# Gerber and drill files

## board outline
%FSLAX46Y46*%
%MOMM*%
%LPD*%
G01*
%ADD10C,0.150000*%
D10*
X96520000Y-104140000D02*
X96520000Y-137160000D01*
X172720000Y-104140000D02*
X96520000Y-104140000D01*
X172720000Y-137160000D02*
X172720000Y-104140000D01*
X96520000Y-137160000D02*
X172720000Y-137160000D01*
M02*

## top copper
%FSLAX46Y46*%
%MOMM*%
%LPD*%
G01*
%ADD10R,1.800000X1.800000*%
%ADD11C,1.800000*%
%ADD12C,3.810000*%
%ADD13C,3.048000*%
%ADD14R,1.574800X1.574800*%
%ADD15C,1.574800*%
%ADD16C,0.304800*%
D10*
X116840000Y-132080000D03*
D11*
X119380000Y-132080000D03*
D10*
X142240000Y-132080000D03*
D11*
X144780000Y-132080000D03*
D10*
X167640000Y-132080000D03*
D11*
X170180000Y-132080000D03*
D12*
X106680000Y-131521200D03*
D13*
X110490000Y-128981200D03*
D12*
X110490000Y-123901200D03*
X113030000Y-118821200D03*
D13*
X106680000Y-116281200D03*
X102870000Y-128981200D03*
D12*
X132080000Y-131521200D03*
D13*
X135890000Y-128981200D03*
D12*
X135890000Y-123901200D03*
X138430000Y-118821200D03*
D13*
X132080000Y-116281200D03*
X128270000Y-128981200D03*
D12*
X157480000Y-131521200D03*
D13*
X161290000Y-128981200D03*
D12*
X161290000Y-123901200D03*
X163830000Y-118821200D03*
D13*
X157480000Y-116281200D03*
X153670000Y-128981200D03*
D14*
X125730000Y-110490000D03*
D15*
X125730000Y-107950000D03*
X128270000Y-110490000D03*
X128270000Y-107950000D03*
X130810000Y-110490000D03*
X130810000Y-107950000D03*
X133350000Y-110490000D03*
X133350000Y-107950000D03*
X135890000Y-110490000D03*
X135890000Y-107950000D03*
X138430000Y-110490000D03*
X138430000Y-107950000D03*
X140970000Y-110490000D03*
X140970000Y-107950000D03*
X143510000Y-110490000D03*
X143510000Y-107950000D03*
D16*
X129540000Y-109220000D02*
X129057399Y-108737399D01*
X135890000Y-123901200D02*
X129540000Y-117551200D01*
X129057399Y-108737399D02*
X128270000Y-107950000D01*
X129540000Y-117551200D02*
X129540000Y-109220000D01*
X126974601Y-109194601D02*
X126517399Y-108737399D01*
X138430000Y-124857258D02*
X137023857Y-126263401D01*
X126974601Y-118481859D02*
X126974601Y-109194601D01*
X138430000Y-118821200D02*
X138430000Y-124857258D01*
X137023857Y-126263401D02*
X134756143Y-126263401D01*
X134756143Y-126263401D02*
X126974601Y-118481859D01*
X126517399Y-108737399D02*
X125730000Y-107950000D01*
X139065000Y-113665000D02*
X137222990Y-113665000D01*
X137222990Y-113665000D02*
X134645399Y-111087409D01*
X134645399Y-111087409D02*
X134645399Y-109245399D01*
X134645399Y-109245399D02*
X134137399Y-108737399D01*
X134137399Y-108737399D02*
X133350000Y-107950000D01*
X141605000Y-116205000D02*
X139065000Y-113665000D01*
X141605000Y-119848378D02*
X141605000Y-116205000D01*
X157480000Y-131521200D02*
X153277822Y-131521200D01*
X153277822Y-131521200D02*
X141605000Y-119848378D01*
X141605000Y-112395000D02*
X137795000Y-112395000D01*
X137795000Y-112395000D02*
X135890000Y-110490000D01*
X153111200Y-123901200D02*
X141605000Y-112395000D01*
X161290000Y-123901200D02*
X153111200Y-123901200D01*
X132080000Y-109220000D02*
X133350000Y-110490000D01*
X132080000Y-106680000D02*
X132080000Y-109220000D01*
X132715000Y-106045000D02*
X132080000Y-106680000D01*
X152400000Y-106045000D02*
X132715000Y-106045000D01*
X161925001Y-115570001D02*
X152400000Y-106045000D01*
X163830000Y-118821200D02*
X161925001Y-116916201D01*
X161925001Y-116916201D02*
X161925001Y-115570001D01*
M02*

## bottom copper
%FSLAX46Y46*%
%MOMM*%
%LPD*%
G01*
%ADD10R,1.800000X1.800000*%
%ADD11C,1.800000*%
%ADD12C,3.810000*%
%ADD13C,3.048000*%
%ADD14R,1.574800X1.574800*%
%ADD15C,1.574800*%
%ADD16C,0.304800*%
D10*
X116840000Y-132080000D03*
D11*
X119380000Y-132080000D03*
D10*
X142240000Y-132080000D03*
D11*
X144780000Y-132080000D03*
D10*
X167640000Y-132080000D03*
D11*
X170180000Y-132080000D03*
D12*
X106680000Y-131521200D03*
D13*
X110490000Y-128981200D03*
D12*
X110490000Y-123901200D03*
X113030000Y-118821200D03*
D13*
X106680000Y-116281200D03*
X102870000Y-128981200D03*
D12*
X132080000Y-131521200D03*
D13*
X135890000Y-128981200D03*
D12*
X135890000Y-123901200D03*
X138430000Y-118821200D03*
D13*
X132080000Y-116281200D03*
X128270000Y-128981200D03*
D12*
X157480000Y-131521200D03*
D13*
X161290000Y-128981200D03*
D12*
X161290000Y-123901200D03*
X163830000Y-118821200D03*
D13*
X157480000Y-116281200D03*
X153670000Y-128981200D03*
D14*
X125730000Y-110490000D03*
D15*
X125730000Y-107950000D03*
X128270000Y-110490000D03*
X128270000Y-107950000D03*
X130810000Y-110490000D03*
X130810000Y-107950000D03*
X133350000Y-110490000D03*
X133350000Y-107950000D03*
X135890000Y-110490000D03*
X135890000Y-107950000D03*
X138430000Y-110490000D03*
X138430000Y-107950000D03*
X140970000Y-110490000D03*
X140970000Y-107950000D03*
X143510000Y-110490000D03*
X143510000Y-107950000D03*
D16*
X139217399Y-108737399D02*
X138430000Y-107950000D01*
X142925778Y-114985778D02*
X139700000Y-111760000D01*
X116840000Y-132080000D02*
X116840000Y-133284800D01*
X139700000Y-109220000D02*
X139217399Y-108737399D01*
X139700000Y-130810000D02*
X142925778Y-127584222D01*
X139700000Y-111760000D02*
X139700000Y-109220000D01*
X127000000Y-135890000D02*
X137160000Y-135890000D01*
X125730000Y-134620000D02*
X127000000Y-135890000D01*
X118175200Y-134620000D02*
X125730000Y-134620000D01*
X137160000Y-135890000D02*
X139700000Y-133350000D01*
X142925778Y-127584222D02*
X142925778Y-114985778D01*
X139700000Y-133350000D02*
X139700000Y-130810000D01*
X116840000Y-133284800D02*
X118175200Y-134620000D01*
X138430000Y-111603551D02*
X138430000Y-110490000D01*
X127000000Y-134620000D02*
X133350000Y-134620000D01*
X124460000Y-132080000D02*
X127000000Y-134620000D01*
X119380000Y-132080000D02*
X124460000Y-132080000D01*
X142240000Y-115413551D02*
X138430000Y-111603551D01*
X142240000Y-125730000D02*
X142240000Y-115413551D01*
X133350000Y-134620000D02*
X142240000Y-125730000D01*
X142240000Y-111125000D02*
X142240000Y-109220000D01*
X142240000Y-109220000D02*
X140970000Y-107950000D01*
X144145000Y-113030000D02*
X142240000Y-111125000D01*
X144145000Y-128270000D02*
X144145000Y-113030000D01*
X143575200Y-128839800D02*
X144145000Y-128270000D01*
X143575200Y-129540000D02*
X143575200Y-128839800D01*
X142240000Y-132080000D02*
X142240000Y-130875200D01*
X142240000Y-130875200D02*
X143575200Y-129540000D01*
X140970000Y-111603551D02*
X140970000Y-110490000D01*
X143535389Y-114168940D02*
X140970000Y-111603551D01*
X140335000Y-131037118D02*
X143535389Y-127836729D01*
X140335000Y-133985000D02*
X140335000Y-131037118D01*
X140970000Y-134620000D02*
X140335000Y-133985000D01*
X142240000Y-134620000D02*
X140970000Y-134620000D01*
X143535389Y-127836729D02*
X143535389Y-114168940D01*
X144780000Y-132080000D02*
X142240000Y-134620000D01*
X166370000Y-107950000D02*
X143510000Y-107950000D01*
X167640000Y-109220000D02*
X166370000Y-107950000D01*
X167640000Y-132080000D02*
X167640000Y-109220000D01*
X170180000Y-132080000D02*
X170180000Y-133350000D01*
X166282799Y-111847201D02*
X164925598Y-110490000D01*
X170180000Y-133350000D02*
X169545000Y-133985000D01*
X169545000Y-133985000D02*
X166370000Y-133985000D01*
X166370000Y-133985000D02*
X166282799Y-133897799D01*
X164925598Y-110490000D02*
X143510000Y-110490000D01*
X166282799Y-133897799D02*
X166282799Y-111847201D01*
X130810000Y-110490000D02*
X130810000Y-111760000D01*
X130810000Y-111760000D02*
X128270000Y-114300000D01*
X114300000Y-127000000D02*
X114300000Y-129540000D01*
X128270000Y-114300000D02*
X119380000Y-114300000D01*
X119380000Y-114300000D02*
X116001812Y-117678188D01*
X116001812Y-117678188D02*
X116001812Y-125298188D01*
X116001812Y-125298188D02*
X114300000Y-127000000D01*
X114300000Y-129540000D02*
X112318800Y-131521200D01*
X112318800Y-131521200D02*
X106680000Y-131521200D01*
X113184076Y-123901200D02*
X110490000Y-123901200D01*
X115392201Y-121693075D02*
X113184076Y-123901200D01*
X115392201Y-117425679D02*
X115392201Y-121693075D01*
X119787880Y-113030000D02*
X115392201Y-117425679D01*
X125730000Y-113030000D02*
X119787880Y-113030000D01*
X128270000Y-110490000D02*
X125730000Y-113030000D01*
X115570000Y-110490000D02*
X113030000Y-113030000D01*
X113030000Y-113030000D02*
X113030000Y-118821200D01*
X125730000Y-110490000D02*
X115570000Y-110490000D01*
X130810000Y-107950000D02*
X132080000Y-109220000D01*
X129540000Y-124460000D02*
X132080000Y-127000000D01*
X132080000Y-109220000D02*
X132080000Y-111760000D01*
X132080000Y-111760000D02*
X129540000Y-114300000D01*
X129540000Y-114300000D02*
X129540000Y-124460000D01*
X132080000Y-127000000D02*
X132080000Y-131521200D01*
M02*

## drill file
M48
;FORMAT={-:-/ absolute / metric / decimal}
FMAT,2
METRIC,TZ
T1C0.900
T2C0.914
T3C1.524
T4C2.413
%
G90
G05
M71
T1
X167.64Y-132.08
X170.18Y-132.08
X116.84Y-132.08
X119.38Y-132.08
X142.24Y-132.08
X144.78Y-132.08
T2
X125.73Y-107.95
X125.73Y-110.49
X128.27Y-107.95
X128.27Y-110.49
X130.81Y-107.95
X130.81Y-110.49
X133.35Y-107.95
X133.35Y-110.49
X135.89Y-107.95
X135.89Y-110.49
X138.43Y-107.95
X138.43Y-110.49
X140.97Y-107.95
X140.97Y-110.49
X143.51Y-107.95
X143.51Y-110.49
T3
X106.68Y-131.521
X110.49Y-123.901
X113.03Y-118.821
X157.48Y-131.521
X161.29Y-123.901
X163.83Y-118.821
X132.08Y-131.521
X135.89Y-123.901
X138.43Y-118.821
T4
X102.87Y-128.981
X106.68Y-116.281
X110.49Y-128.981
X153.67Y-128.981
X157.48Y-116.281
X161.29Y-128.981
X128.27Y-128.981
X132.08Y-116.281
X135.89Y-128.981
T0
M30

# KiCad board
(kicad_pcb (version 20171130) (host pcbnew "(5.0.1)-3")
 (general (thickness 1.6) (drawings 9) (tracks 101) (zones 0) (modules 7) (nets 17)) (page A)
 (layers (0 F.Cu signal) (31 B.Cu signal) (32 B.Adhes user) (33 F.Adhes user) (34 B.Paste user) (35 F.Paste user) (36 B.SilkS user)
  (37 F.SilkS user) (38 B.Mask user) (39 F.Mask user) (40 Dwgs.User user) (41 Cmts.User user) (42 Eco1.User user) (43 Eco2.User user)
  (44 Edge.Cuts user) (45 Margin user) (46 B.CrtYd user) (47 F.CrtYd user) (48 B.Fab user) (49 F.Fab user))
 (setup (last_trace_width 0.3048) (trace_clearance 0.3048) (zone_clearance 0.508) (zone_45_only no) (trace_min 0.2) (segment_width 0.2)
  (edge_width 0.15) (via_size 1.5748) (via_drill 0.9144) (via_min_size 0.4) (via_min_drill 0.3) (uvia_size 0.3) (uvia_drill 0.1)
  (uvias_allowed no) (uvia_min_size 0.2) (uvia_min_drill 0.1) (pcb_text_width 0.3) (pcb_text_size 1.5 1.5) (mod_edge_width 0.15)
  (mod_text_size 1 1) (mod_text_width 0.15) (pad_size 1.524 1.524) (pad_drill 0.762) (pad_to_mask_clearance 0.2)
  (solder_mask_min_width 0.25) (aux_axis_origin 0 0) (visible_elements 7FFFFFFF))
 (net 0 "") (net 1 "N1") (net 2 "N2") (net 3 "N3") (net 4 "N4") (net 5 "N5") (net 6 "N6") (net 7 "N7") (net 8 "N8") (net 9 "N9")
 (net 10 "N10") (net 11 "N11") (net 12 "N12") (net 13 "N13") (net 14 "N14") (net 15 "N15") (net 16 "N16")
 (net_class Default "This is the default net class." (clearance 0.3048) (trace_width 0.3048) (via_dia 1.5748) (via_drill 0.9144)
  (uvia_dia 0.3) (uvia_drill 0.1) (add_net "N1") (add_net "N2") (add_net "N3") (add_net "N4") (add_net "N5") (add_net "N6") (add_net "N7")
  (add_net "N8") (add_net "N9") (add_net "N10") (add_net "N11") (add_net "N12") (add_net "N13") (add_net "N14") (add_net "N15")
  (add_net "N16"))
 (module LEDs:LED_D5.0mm (layer F.Cu) (at 116.84 132.08)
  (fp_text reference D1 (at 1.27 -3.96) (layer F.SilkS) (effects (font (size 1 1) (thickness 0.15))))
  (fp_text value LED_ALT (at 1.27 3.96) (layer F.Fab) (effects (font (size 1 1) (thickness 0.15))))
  (pad 1 thru_hole rect (at 0 0) (size 1.8 1.8) (drill 0.9) (layers *.Cu *.Mask) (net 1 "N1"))
  (pad 2 thru_hole circle (at 2.54 0) (size 1.8 1.8) (drill 0.9) (layers *.Cu *.Mask) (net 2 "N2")))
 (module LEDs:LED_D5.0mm (layer F.Cu) (at 142.24 132.08)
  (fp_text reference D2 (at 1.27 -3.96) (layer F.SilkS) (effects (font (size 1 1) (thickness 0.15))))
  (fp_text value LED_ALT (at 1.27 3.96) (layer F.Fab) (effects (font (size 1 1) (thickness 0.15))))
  (pad 1 thru_hole rect (at 0 0) (size 1.8 1.8) (drill 0.9) (layers *.Cu *.Mask) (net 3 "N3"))
  (pad 2 thru_hole circle (at 2.54 0) (size 1.8 1.8) (drill 0.9) (layers *.Cu *.Mask) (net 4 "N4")))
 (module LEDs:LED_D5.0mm (layer F.Cu) (at 167.64 132.08)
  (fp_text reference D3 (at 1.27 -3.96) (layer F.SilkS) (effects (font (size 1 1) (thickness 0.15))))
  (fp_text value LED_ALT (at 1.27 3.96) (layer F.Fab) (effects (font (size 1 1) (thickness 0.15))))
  (pad 1 thru_hole rect (at 0 0) (size 1.8 1.8) (drill 0.9) (layers *.Cu *.Mask) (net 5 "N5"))
  (pad 2 thru_hole circle (at 2.54 0) (size 1.8 1.8) (drill 0.9) (layers *.Cu *.Mask) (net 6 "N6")))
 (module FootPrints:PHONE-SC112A (layer F.Cu) (at 106.68 137.16 270)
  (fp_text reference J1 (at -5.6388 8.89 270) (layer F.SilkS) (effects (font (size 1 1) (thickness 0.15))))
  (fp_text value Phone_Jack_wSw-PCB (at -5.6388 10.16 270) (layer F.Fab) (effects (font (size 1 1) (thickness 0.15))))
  (pad 1 thru_hole circle (at -5.6388 0 270) (size 3.81 3.81) (drill 1.524) (layers *.Cu *.Mask F.SilkS) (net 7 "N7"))
  (pad "" thru_hole circle (at -8.1788 -3.81 270) (size 3.048 3.048) (drill 2.413) (layers *.Cu *.Mask F.SilkS))
  (pad 2 thru_hole circle (at -13.2588 -3.81 270) (size 3.81 3.81) (drill 1.524) (layers *.Cu *.Mask F.SilkS) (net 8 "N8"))
  (pad 3 thru_hole circle (at -18.3388 -6.35 270) (size 3.81 3.81) (drill 1.524) (layers *.Cu *.Mask F.SilkS) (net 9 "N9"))
  (pad "" thru_hole circle (at -20.8788 0 270) (size 3.048 3.048) (drill 2.413) (layers *.Cu *.Mask F.SilkS))
  (pad "" thru_hole circle (at -8.1788 3.81 270) (size 3.048 3.048) (drill 2.413) (layers *.Cu *.Mask F.SilkS)))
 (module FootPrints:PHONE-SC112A (layer F.Cu) (at 132.08 137.16 270)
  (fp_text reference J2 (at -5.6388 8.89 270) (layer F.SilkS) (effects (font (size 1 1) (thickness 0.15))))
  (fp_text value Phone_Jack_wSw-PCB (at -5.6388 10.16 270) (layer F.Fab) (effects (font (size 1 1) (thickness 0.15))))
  (pad 1 thru_hole circle (at -5.6388 0 270) (size 3.81 3.81) (drill 1.524) (layers *.Cu *.Mask F.SilkS) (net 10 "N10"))
  (pad "" thru_hole circle (at -8.1788 -3.81 270) (size 3.048 3.048) (drill 2.413) (layers *.Cu *.Mask F.SilkS))
  (pad 2 thru_hole circle (at -13.2588 -3.81 270) (size 3.81 3.81) (drill 1.524) (layers *.Cu *.Mask F.SilkS) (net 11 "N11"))
  (pad 3 thru_hole circle (at -18.3388 -6.35 270) (size 3.81 3.81) (drill 1.524) (layers *.Cu *.Mask F.SilkS) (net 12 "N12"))
  (pad "" thru_hole circle (at -20.8788 0 270) (size 3.048 3.048) (drill 2.413) (layers *.Cu *.Mask F.SilkS))
  (pad "" thru_hole circle (at -8.1788 3.81 270) (size 3.048 3.048) (drill 2.413) (layers *.Cu *.Mask F.SilkS)))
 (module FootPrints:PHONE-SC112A (layer F.Cu) (at 157.48 137.16 270)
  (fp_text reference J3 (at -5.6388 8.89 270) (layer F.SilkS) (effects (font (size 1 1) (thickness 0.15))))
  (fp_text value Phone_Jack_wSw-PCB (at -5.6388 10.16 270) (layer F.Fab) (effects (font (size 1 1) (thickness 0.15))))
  (pad 1 thru_hole circle (at -5.6388 0 270) (size 3.81 3.81) (drill 1.524) (layers *.Cu *.Mask F.SilkS) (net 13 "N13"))
  (pad "" thru_hole circle (at -8.1788 -3.81 270) (size 3.048 3.048) (drill 2.413) (layers *.Cu *.Mask F.SilkS))
  (pad 2 thru_hole circle (at -13.2588 -3.81 270) (size 3.81 3.81) (drill 1.524) (layers *.Cu *.Mask F.SilkS) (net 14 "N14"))
  (pad 3 thru_hole circle (at -18.3388 -6.35 270) (size 3.81 3.81) (drill 1.524) (layers *.Cu *.Mask F.SilkS) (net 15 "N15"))
  (pad "" thru_hole circle (at -20.8788 0 270) (size 3.048 3.048) (drill 2.413) (layers *.Cu *.Mask F.SilkS))
  (pad "" thru_hole circle (at -8.1788 3.81 270) (size 3.048 3.048) (drill 2.413) (layers *.Cu *.Mask F.SilkS)))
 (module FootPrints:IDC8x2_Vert (layer F.Cu) (at 134.62 109.22 180)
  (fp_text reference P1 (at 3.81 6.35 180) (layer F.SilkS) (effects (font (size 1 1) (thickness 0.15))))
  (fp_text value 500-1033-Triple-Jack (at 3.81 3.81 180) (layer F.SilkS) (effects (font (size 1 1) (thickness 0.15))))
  (pad 1 thru_hole rect (at 8.89 -1.27 180) (size 1.5748 1.5748) (drill 0.9144) (layers *.Cu *.Mask F.SilkS) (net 9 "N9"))
  (pad 2 thru_hole circle (at 8.89 1.27 180) (size 1.5748 1.5748) (drill 0.9144) (layers *.Cu *.Mask F.SilkS) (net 12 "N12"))
  (pad 3 thru_hole circle (at 6.35 -1.27 180) (size 1.5748 1.5748) (drill 0.9144) (layers *.Cu *.Mask F.SilkS) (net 8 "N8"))
  (pad 4 thru_hole circle (at 6.35 1.27 180) (size 1.5748 1.5748) (drill 0.9144) (layers *.Cu *.Mask F.SilkS) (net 11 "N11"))
  (pad 5 thru_hole circle (at 3.81 -1.27 180) (size 1.5748 1.5748) (drill 0.9144) (layers *.Cu *.Mask F.SilkS) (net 7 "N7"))
  (pad 6 thru_hole circle (at 3.81 1.27 180) (size 1.5748 1.5748) (drill 0.9144) (layers *.Cu *.Mask F.SilkS) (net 10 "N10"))
  (pad 7 thru_hole circle (at 1.27 -1.27 180) (size 1.5748 1.5748) (drill 0.9144) (layers *.Cu *.Mask F.SilkS) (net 15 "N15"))
  (pad 8 thru_hole circle (at 1.27 1.27 180) (size 1.5748 1.5748) (drill 0.9144) (layers *.Cu *.Mask F.SilkS) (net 13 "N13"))
  (pad 9 thru_hole circle (at -1.27 -1.27 180) (size 1.5748 1.5748) (drill 0.9144) (layers *.Cu *.Mask F.SilkS) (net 14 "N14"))
  (pad 10 thru_hole circle (at -1.27 1.27 180) (size 1.5748 1.5748) (drill 0.9144) (layers *.Cu *.Mask F.SilkS) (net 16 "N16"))
  (pad 11 thru_hole circle (at -3.81 -1.27 180) (size 1.5748 1.5748) (drill 0.9144) (layers *.Cu *.Mask F.SilkS) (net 2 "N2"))
  (pad 12 thru_hole circle (at -3.81 1.27 180) (size 1.5748 1.5748) (drill 0.9144) (layers *.Cu *.Mask F.SilkS) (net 1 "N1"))
  (pad 13 thru_hole circle (at -6.35 -1.27 180) (size 1.5748 1.5748) (drill 0.9144) (layers *.Cu *.Mask F.SilkS) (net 4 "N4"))
  (pad 14 thru_hole circle (at -6.35 1.27 180) (size 1.5748 1.5748) (drill 0.9144) (layers *.Cu *.Mask F.SilkS) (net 3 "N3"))
  (pad 15 thru_hole circle (at -8.89 -1.27 180) (size 1.5748 1.5748) (drill 0.9144) (layers *.Cu *.Mask F.SilkS) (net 6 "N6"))
  (pad 16 thru_hole circle (at -8.89 1.27 180) (size 1.5748 1.5748) (drill 0.9144) (layers *.Cu *.Mask F.SilkS) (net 5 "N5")))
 (gr_line (start 96.52 104.14) (end 96.52 137.16) (angle 90) (layer Edge.Cuts) (width 0.15))
 (gr_line (start 172.72 104.14) (end 96.52 104.14) (angle 90) (layer Edge.Cuts) (width 0.15))
 (gr_line (start 172.72 137.16) (end 172.72 104.14) (angle 90) (layer Edge.Cuts) (width 0.15))
 (gr_line (start 96.52 137.16) (end 172.72 137.16) (angle 90) (layer Edge.Cuts) (width 0.15))
 (segment (start 139.217399 108.737399) (end 138.43 107.95) (width 0.3048) (layer B.Cu) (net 1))
 (segment (start 142.925778 114.985778) (end 139.7 111.76) (width 0.3048) (layer B.Cu) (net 1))
 (segment (start 116.84 132.08) (end 116.84 133.2848) (width 0.3048) (layer B.Cu) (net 1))
 (segment (start 139.7 109.22) (end 139.217399 108.737399) (width 0.3048) (layer B.Cu) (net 1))
 (segment (start 139.7 130.81) (end 142.925778 127.584222) (width 0.3048) (layer B.Cu) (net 1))
 (segment (start 139.7 111.76) (end 139.7 109.22) (width 0.3048) (layer B.Cu) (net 1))
 (segment (start 127 135.89) (end 137.16 135.89) (width 0.3048) (layer B.Cu) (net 1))
 (segment (start 125.73 134.62) (end 127 135.89) (width 0.3048) (layer B.Cu) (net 1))
 (segment (start 118.1752 134.62) (end 125.73 134.62) (width 0.3048) (layer B.Cu) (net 1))
 (segment (start 137.16 135.89) (end 139.7 133.35) (width 0.3048) (layer B.Cu) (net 1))
 (segment (start 142.925778 127.584222) (end 142.925778 114.985778) (width 0.3048) (layer B.Cu) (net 1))
 (segment (start 139.7 133.35) (end 139.7 130.81) (width 0.3048) (layer B.Cu) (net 1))
 (segment (start 116.84 133.2848) (end 118.1752 134.62) (width 0.3048) (layer B.Cu) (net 1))
 (segment (start 138.43 111.603551) (end 138.43 110.49) (width 0.3048) (layer B.Cu) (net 2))
 (segment (start 127 134.62) (end 133.35 134.62) (width 0.3048) (layer B.Cu) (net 2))
 (segment (start 124.46 132.08) (end 127 134.62) (width 0.3048) (layer B.Cu) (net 2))
 (segment (start 119.38 132.08) (end 124.46 132.08) (width 0.3048) (layer B.Cu) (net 2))
 (segment (start 142.24 115.413551) (end 138.43 111.603551) (width 0.3048) (layer B.Cu) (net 2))
 (segment (start 142.24 125.73) (end 142.24 115.413551) (width 0.3048) (layer B.Cu) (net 2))
 (segment (start 133.35 134.62) (end 142.24 125.73) (width 0.3048) (layer B.Cu) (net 2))
 (segment (start 142.24 111.125) (end 142.24 109.22) (width 0.3048) (layer B.Cu) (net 3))
 (segment (start 142.24 109.22) (end 140.97 107.95) (width 0.3048) (layer B.Cu) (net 3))
 (segment (start 144.145 113.03) (end 142.24 111.125) (width 0.3048) (layer B.Cu) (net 3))
 (segment (start 144.145 128.27) (end 144.145 113.03) (width 0.3048) (layer B.Cu) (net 3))
 (segment (start 143.5752 128.8398) (end 144.145 128.27) (width 0.3048) (layer B.Cu) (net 3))
 (segment (start 143.5752 129.54) (end 143.5752 128.8398) (width 0.3048) (layer B.Cu) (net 3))
 (segment (start 142.24 132.08) (end 142.24 130.8752) (width 0.3048) (layer B.Cu) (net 3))
 (segment (start 142.24 130.8752) (end 143.5752 129.54) (width 0.3048) (layer B.Cu) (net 3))
 (segment (start 140.97 111.603551) (end 140.97 110.49) (width 0.3048) (layer B.Cu) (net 4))
 (segment (start 143.535389 114.16894) (end 140.97 111.603551) (width 0.3048) (layer B.Cu) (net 4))
 (segment (start 140.335 131.037118) (end 143.535389 127.836729) (width 0.3048) (layer B.Cu) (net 4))
 (segment (start 140.335 133.985) (end 140.335 131.037118) (width 0.3048) (layer B.Cu) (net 4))
 (segment (start 140.97 134.62) (end 140.335 133.985) (width 0.3048) (layer B.Cu) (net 4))
 (segment (start 142.24 134.62) (end 140.97 134.62) (width 0.3048) (layer B.Cu) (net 4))
 (segment (start 143.535389 127.836729) (end 143.535389 114.16894) (width 0.3048) (layer B.Cu) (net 4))
 (segment (start 144.78 132.08) (end 142.24 134.62) (width 0.3048) (layer B.Cu) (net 4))
 (segment (start 166.37 107.95) (end 143.51 107.95) (width 0.3048) (layer B.Cu) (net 5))
 (segment (start 167.64 109.22) (end 166.37 107.95) (width 0.3048) (layer B.Cu) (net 5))
 (segment (start 167.64 132.08) (end 167.64 109.22) (width 0.3048) (layer B.Cu) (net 5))
 (segment (start 170.18 132.08) (end 170.18 133.35) (width 0.3048) (layer B.Cu) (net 6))
 (segment (start 166.282799 111.847201) (end 164.925598 110.49) (width 0.3048) (layer B.Cu) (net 6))
 (segment (start 170.18 133.35) (end 169.545 133.985) (width 0.3048) (layer B.Cu) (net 6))
 (segment (start 169.545 133.985) (end 166.37 133.985) (width 0.3048) (layer B.Cu) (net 6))
 (segment (start 166.37 133.985) (end 166.282799 133.897799) (width 0.3048) (layer B.Cu) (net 6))
 (segment (start 164.925598 110.49) (end 143.51 110.49) (width 0.3048) (layer B.Cu) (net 6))
 (segment (start 166.282799 133.897799) (end 166.282799 111.847201) (width 0.3048) (layer B.Cu) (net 6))
 (segment (start 130.81 110.49) (end 130.81 111.76) (width 0.3048) (layer B.Cu) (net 7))
 (segment (start 130.81 111.76) (end 128.27 114.3) (width 0.3048) (layer B.Cu) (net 7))
 (segment (start 114.3 127) (end 114.3 129.54) (width 0.3048) (layer B.Cu) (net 7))
 (segment (start 128.27 114.3) (end 119.38 114.3) (width 0.3048) (layer B.Cu) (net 7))
 (segment (start 119.38 114.3) (end 116.001812 117.678188) (width 0.3048) (layer B.Cu) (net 7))
 (segment (start 116.001812 117.678188) (end 116.001812 125.298188) (width 0.3048) (layer B.Cu) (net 7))
 (segment (start 116.001812 125.298188) (end 114.3 127) (width 0.3048) (layer B.Cu) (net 7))
 (segment (start 114.3 129.54) (end 112.3188 131.5212) (width 0.3048) (layer B.Cu) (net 7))
 (segment (start 112.3188 131.5212) (end 106.68 131.5212) (width 0.3048) (layer B.Cu) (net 7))
 (segment (start 113.184076 123.9012) (end 110.49 123.9012) (width 0.3048) (layer B.Cu) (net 8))
 (segment (start 115.392201 121.693075) (end 113.184076 123.9012) (width 0.3048) (layer B.Cu) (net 8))
 (segment (start 115.392201 117.425679) (end 115.392201 121.693075) (width 0.3048) (layer B.Cu) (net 8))
 (segment (start 119.78788 113.03) (end 115.392201 117.425679) (width 0.3048) (layer B.Cu) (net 8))
 (segment (start 125.73 113.03) (end 119.78788 113.03) (width 0.3048) (layer B.Cu) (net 8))
 (segment (start 128.27 110.49) (end 125.73 113.03) (width 0.3048) (layer B.Cu) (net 8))
 (segment (start 115.57 110.49) (end 113.03 113.03) (width 0.3048) (layer B.Cu) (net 9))
 (segment (start 113.03 113.03) (end 113.03 118.8212) (width 0.3048) (layer B.Cu) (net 9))
 (segment (start 125.73 110.49) (end 115.57 110.49) (width 0.3048) (layer B.Cu) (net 9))
 (segment (start 130.81 107.95) (end 132.08 109.22) (width 0.3048) (layer B.Cu) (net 10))
 (segment (start 129.54 124.46) (end 132.08 127) (width 0.3048) (layer B.Cu) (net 10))
 (segment (start 132.08 109.22) (end 132.08 111.76) (width 0.3048) (layer B.Cu) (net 10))
 (segment (start 132.08 111.76) (end 129.54 114.3) (width 0.3048) (layer B.Cu) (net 10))
 (segment (start 129.54 114.3) (end 129.54 124.46) (width 0.3048) (layer B.Cu) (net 10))
 (segment (start 132.08 127) (end 132.08 131.5212) (width 0.3048) (layer B.Cu) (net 10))
 (segment (start 129.54 109.22) (end 129.057399 108.737399) (width 0.3048) (layer F.Cu) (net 11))
 (segment (start 135.89 123.9012) (end 129.54 117.5512) (width 0.3048) (layer F.Cu) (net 11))
 (segment (start 129.057399 108.737399) (end 128.27 107.95) (width 0.3048) (layer F.Cu) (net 11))
 (segment (start 129.54 117.5512) (end 129.54 109.22) (width 0.3048) (layer F.Cu) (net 11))
 (segment (start 126.974601 109.194601) (end 126.517399 108.737399) (width 0.3048) (layer F.Cu) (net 12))
 (segment (start 138.43 124.857258) (end 137.023857 126.263401) (width 0.3048) (layer F.Cu) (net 12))
 (segment (start 126.974601 118.481859) (end 126.974601 109.194601) (width 0.3048) (layer F.Cu) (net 12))
 (segment (start 138.43 118.8212) (end 138.43 124.857258) (width 0.3048) (layer F.Cu) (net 12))
 (segment (start 137.023857 126.263401) (end 134.756143 126.263401) (width 0.3048) (layer F.Cu) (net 12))
 (segment (start 134.756143 126.263401) (end 126.974601 118.481859) (width 0.3048) (layer F.Cu) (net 12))
 (segment (start 126.517399 108.737399) (end 125.73 107.95) (width 0.3048) (layer F.Cu) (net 12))
 (segment (start 139.065 113.665) (end 137.22299 113.665) (width 0.3048) (layer F.Cu) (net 13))
 (segment (start 137.22299 113.665) (end 134.645399 111.087409) (width 0.3048) (layer F.Cu) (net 13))
 (segment (start 134.645399 111.087409) (end 134.645399 109.245399) (width 0.3048) (layer F.Cu) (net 13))
 (segment (start 134.645399 109.245399) (end 134.137399 108.737399) (width 0.3048) (layer F.Cu) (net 13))
 (segment (start 134.137399 108.737399) (end 133.35 107.95) (width 0.3048) (layer F.Cu) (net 13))
 (segment (start 141.605 116.205) (end 139.065 113.665) (width 0.3048) (layer F.Cu) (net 13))
 (segment (start 141.605 119.848378) (end 141.605 116.205) (width 0.3048) (layer F.Cu) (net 13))
 (segment (start 157.48 131.5212) (end 153.277822 131.5212) (width 0.3048) (layer F.Cu) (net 13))
 (segment (start 153.277822 131.5212) (end 141.605 119.848378) (width 0.3048) (layer F.Cu) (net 13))
 (segment (start 141.605 112.395) (end 137.795 112.395) (width 0.3048) (layer F.Cu) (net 14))
 (segment (start 137.795 112.395) (end 135.89 110.49) (width 0.3048) (layer F.Cu) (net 14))
 (segment (start 153.1112 123.9012) (end 141.605 112.395) (width 0.3048) (layer F.Cu) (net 14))
 (segment (start 161.29 123.9012) (end 153.1112 123.9012) (width 0.3048) (layer F.Cu) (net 14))
 (segment (start 132.08 109.22) (end 133.35 110.49) (width 0.3048) (layer F.Cu) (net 15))
 (segment (start 132.08 106.68) (end 132.08 109.22) (width 0.3048) (layer F.Cu) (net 15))
 (segment (start 132.715 106.045) (end 132.08 106.68) (width 0.3048) (layer F.Cu) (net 15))
 (segment (start 152.4 106.045) (end 132.715 106.045) (width 0.3048) (layer F.Cu) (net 15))
 (segment (start 161.925001 115.570001) (end 152.4 106.045) (width 0.3048) (layer F.Cu) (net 15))
 (segment (start 163.83 118.8212) (end 161.925001 116.916201) (width 0.3048) (layer F.Cu) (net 15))
 (segment (start 161.925001 116.916201) (end 161.925001 115.570001) (width 0.3048) (layer F.Cu) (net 15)))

